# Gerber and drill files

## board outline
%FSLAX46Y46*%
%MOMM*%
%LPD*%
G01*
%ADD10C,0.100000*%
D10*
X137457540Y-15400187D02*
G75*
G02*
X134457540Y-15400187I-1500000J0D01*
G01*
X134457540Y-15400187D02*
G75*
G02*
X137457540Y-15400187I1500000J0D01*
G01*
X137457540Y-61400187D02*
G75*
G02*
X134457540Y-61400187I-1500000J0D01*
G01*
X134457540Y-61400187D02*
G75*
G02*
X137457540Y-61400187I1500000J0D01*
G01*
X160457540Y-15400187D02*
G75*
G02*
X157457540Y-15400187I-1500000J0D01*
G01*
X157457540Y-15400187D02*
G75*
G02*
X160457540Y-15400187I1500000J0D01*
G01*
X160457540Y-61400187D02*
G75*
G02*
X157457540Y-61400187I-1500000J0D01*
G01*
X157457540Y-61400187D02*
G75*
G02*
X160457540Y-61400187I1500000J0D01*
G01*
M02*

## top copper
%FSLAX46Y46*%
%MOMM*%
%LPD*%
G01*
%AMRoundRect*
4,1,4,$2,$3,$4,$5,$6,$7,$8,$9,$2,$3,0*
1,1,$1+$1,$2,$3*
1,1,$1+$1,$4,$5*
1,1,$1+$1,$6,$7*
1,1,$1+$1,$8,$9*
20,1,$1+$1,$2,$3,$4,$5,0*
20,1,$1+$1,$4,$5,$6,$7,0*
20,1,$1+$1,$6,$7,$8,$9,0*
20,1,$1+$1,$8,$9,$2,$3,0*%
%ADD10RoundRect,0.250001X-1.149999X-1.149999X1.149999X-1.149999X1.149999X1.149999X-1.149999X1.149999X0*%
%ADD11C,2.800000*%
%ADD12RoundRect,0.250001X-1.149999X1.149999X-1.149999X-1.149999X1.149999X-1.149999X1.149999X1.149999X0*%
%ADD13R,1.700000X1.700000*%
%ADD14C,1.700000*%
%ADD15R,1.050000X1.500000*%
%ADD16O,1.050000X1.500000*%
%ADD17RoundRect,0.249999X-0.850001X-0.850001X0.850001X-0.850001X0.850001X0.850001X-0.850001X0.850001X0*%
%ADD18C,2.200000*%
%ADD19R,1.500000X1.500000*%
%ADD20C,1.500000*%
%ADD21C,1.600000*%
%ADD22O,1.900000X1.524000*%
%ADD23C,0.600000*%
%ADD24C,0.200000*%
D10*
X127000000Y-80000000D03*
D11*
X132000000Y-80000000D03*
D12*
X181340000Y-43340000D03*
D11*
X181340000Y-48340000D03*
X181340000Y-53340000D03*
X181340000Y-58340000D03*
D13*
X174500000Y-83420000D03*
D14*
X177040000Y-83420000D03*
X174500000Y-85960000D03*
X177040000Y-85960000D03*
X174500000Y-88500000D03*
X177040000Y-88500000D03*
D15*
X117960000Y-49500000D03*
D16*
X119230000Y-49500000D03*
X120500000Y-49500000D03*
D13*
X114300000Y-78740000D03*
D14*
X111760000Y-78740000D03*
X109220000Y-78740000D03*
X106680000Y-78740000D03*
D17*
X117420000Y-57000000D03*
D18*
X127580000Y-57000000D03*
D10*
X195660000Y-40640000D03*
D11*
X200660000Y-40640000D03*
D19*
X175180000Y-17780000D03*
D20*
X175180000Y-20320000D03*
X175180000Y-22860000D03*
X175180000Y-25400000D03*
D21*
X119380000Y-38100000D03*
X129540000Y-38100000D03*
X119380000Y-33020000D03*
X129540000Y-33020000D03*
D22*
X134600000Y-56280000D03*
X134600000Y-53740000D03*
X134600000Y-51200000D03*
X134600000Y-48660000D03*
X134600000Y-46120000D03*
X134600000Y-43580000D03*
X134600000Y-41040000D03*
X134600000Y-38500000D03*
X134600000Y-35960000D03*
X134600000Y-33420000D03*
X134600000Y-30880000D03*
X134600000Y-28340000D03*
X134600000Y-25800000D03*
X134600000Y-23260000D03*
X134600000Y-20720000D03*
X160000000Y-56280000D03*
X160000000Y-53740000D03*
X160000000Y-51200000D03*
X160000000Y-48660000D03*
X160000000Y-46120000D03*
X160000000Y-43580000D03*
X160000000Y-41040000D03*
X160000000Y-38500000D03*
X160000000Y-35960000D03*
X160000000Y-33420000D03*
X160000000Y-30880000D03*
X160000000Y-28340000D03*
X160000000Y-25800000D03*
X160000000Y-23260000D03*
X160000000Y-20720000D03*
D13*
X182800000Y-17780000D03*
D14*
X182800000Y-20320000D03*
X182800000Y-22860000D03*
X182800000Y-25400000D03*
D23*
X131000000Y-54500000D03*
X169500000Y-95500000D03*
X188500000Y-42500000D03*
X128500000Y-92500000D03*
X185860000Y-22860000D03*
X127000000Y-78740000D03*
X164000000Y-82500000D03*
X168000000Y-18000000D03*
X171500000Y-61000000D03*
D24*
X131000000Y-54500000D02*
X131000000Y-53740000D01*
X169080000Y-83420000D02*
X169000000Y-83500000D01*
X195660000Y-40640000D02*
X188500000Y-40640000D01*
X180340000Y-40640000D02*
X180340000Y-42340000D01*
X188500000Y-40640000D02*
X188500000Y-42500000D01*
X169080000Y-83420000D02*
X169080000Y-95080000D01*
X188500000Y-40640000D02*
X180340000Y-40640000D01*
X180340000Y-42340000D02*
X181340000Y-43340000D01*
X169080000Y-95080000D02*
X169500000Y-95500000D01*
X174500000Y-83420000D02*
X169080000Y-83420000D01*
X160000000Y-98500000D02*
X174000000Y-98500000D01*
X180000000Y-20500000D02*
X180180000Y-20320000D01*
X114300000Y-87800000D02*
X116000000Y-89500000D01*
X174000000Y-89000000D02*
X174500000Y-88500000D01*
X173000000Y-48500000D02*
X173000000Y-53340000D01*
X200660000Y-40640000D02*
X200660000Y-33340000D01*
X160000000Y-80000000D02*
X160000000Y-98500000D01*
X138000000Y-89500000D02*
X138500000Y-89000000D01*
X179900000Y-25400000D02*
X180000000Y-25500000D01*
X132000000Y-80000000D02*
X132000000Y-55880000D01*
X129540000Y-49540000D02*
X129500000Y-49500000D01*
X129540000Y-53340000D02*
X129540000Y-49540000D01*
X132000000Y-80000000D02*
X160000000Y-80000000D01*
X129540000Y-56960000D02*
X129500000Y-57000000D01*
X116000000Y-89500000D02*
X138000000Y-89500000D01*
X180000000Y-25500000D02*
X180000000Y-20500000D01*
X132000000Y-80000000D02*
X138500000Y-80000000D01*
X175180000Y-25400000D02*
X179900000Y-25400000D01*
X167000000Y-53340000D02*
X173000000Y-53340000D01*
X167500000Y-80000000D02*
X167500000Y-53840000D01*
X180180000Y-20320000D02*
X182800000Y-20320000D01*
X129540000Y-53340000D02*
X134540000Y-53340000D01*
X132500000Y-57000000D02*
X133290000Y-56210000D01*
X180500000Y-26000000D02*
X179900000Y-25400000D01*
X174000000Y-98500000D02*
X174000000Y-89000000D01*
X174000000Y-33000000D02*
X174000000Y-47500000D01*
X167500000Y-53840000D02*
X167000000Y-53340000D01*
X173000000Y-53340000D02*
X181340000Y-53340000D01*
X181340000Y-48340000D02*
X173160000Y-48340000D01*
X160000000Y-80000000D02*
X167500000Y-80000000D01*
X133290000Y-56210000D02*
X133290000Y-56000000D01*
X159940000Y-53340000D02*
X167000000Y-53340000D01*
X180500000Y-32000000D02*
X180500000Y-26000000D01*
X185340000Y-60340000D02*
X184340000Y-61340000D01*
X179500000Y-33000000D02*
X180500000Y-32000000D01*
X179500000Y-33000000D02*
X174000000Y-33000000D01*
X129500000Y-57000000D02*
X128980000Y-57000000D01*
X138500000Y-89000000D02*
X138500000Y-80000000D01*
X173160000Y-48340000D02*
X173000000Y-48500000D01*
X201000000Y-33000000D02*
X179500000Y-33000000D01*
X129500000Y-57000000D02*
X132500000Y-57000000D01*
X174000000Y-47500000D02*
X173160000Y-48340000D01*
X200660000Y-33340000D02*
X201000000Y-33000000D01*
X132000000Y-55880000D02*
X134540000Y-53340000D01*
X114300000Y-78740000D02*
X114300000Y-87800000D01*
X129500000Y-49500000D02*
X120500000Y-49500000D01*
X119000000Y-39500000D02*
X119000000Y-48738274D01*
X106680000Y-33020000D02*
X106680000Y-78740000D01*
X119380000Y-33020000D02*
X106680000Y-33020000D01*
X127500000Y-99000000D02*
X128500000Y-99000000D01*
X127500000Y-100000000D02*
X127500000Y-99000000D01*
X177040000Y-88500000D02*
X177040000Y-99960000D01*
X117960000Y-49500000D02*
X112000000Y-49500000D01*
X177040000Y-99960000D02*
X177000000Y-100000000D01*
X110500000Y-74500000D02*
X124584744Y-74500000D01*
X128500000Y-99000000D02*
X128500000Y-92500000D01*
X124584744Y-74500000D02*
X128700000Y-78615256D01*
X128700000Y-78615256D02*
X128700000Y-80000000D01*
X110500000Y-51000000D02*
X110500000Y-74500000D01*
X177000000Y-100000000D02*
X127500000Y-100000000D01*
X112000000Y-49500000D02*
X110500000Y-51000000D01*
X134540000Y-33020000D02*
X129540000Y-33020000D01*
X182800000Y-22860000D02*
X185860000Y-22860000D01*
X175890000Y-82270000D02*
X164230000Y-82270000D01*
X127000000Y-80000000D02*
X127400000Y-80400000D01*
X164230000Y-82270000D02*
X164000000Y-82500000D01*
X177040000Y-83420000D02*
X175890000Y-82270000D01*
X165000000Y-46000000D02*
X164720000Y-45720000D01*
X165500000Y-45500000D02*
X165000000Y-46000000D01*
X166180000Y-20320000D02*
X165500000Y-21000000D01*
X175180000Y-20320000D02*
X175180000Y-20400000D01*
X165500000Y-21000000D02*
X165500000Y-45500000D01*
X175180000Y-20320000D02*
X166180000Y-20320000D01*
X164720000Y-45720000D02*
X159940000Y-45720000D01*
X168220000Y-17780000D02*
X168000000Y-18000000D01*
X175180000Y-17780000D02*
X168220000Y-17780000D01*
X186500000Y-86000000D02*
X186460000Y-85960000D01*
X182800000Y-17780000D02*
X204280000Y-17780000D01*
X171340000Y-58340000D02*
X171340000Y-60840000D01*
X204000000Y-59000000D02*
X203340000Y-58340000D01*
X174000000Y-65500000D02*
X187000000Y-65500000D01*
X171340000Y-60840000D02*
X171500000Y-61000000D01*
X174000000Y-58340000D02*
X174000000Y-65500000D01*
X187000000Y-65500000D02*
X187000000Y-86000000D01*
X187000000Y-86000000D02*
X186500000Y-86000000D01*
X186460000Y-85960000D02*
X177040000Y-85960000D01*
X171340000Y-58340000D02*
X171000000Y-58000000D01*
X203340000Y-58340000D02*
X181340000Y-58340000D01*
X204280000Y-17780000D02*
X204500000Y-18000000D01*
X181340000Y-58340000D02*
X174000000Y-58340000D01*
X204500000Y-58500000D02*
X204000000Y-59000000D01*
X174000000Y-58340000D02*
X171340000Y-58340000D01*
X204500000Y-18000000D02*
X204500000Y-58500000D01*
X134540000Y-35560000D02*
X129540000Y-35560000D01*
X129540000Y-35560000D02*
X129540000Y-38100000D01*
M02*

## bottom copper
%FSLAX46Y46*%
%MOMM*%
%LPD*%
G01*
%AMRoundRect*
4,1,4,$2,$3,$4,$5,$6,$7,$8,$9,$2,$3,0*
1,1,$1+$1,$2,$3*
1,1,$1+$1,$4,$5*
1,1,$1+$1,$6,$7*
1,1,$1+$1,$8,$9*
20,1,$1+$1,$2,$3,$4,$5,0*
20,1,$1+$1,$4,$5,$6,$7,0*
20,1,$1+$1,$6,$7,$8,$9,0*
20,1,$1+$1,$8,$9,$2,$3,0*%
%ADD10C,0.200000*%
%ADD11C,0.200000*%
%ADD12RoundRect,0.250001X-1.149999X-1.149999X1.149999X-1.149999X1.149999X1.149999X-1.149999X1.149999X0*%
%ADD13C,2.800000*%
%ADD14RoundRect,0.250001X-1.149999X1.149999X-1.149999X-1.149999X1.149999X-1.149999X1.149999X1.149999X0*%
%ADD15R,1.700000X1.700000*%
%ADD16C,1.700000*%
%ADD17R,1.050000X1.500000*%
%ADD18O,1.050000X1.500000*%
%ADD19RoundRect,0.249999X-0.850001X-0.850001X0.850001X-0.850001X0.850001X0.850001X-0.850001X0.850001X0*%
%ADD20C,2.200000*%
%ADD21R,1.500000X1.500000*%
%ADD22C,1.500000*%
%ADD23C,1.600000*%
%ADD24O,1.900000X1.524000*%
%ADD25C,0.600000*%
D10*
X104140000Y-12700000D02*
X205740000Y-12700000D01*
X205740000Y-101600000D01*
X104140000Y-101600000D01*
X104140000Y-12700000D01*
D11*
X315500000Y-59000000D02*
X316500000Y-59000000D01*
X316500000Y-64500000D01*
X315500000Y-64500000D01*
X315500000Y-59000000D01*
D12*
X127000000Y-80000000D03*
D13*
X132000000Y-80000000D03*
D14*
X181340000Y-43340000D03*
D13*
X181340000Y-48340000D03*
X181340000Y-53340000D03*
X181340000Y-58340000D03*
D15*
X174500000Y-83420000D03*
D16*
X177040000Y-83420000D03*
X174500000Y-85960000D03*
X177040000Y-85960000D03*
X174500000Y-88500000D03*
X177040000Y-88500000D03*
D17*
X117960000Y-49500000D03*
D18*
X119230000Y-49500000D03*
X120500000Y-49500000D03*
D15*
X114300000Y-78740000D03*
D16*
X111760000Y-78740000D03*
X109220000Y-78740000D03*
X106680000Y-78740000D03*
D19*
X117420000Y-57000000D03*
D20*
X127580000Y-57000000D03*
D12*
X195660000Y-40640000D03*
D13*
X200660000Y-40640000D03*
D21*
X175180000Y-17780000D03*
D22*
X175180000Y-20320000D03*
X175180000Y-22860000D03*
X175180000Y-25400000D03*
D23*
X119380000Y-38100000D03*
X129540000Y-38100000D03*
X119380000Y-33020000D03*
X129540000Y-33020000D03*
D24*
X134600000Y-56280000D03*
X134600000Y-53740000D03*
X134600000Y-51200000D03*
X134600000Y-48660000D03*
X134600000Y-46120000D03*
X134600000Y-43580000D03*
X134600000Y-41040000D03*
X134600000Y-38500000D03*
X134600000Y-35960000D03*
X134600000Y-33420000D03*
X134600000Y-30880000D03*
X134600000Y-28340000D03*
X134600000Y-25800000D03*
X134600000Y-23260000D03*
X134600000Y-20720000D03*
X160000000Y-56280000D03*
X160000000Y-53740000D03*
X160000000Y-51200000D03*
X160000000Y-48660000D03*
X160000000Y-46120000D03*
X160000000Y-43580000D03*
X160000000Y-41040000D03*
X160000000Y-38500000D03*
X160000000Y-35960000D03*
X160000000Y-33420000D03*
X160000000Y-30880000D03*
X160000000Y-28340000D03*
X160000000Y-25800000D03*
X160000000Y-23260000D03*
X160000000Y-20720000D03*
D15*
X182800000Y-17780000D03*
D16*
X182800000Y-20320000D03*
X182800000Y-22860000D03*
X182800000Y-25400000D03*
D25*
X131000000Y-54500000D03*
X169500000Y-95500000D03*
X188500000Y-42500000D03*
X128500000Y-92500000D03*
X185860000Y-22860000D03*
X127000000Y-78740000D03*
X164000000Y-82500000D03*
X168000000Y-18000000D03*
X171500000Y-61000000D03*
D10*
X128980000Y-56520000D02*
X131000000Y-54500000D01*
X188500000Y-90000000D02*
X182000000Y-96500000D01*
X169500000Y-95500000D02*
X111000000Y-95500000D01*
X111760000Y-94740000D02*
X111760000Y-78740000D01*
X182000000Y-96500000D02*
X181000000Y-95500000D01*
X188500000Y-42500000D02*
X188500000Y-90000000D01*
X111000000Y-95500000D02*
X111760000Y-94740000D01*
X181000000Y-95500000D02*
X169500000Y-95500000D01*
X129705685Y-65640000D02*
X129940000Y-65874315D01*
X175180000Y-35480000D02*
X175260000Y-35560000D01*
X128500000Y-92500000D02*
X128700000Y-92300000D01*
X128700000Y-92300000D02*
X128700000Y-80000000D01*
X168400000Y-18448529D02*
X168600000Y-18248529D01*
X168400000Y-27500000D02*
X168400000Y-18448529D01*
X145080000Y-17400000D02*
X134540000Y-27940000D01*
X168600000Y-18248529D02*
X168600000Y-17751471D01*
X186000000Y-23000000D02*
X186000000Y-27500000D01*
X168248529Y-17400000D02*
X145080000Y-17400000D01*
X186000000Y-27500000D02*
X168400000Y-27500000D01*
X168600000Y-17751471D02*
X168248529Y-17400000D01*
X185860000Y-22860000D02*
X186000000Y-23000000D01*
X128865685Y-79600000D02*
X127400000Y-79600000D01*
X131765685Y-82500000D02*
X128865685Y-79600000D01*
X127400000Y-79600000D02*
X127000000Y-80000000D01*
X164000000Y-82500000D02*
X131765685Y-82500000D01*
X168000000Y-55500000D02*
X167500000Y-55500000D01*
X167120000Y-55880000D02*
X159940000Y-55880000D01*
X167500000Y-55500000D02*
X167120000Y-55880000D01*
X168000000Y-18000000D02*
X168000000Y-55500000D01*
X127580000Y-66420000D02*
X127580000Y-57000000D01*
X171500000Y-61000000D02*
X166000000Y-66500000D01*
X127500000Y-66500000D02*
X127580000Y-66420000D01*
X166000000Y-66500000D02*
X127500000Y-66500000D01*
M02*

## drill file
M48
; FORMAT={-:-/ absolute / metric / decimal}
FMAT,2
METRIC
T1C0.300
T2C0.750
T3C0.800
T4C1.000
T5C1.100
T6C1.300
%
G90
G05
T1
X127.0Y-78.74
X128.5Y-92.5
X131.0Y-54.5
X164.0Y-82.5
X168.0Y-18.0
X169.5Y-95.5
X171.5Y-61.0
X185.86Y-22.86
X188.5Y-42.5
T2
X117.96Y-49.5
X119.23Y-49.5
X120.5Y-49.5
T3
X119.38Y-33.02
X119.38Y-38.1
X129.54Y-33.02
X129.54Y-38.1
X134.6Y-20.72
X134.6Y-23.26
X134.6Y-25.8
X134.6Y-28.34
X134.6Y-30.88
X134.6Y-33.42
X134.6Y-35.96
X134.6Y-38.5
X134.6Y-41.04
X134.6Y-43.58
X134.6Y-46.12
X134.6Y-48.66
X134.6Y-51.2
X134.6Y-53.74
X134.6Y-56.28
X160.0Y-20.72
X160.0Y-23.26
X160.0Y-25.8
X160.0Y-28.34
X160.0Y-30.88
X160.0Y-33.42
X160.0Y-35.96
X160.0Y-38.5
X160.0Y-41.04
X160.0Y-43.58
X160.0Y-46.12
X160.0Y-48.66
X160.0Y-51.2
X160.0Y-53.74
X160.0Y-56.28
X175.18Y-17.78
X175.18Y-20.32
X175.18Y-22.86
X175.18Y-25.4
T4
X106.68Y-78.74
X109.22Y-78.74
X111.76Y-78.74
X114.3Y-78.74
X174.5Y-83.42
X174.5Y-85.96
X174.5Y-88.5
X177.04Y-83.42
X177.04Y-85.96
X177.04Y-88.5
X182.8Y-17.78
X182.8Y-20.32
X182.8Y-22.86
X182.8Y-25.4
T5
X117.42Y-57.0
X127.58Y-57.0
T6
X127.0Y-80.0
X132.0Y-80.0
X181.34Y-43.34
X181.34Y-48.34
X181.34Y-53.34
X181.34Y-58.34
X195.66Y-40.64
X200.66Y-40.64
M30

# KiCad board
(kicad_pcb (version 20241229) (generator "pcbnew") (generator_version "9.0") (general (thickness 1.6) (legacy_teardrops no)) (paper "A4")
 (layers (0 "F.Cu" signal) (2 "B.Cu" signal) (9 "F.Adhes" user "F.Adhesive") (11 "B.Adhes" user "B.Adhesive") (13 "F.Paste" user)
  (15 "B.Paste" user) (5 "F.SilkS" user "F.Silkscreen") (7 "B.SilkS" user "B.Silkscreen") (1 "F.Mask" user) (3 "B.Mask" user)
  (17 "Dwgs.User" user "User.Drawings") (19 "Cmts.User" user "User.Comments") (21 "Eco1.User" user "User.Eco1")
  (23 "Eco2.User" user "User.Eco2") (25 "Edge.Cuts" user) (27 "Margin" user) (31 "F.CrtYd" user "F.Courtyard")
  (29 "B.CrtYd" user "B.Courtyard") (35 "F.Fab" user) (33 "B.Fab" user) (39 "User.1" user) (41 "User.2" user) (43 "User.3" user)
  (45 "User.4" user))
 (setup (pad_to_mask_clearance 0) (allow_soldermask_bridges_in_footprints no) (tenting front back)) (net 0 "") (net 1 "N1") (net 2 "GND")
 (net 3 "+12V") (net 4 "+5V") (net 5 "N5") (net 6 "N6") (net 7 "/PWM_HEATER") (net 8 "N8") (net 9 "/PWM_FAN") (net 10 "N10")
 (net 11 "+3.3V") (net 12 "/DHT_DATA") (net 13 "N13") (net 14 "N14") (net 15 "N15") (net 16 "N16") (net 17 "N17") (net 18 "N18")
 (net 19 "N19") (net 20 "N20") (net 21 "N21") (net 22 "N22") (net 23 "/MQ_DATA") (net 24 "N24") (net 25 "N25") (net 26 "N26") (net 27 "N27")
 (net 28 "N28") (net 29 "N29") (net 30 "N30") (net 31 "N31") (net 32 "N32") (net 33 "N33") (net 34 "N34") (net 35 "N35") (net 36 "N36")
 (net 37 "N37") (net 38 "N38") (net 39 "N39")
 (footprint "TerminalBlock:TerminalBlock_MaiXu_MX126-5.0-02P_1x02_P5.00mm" (layer "F.Cu") (at 127 80)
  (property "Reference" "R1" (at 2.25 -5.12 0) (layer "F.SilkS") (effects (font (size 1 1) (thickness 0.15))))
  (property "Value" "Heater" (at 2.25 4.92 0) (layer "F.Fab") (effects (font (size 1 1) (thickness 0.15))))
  (pad "1" thru_hole roundrect (at 0 0) (size 2.8 2.8) (drill 1.3) (layers "*.Cu" "*.Mask") (remove_unused_layers no)
   (roundrect_rratio 0.089286) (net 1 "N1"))
  (pad "2" thru_hole circle (at 5 0) (size 2.8 2.8) (drill 1.3) (layers "*.Cu" "*.Mask") (remove_unused_layers no) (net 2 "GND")))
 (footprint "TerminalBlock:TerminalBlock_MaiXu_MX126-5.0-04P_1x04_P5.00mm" (layer "F.Cu") (at 181.34 43.34 -90)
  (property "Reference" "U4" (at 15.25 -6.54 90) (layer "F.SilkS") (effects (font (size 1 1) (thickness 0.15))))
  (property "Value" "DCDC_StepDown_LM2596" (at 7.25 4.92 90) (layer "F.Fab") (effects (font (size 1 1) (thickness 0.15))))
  (pad "1" thru_hole roundrect (at 0 0 270) (size 2.8 2.8) (drill 1.3) (layers "*.Cu" "*.Mask") (remove_unused_layers no)
   (roundrect_rratio 0.089286) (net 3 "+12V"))
  (pad "2" thru_hole circle (at 5 0 270) (size 2.8 2.8) (drill 1.3) (layers "*.Cu" "*.Mask") (remove_unused_layers no) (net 2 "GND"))
  (pad "3" thru_hole circle (at 10 0 270) (size 2.8 2.8) (drill 1.3) (layers "*.Cu" "*.Mask") (remove_unused_layers no) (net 2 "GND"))
  (pad "4" thru_hole circle (at 15 0 270) (size 2.8 2.8) (drill 1.3) (layers "*.Cu" "*.Mask") (remove_unused_layers no) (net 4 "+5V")))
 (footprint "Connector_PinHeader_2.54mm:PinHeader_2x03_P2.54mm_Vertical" (layer "F.Cu") (at 174.5 83.42)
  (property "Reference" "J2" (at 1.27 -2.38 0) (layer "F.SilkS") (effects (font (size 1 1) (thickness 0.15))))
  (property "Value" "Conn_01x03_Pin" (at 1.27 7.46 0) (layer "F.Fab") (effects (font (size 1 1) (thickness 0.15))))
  (pad "1" thru_hole rect (at 0 0) (size 1.7 1.7) (drill 1) (layers "*.Cu" "*.Mask") (remove_unused_layers no) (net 3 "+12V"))
  (pad "2" thru_hole circle (at 2.54 0) (size 1.7 1.7) (drill 1) (layers "*.Cu" "*.Mask") (remove_unused_layers no) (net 1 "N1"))
  (pad "3" thru_hole circle (at 0 2.54) (size 1.7 1.7) (drill 1) (layers "*.Cu" "*.Mask") (remove_unused_layers no) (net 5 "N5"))
  (pad "4" thru_hole circle (at 2.54 2.54) (size 1.7 1.7) (drill 1) (layers "*.Cu" "*.Mask") (remove_unused_layers no) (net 4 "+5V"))
  (pad "5" thru_hole circle (at 0 5.08) (size 1.7 1.7) (drill 1) (layers "*.Cu" "*.Mask") (remove_unused_layers no) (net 2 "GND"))
  (pad "6" thru_hole circle (at 2.54 5.08) (size 1.7 1.7) (drill 1) (layers "*.Cu" "*.Mask") (remove_unused_layers no) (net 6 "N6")))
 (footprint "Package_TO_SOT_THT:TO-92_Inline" (layer "F.Cu") (at 117.96 49.5)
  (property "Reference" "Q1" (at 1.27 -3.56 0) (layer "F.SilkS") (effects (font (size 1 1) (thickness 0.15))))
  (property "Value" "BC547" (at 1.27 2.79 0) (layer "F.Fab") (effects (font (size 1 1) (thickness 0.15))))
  (pad "1" thru_hole rect (at 0 0) (size 1.05 1.5) (drill 0.75) (layers "*.Cu" "*.Mask") (remove_unused_layers no) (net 6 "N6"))
  (pad "2" thru_hole oval (at 1.27 0) (size 1.05 1.5) (drill 0.75) (layers "*.Cu" "*.Mask") (remove_unused_layers no) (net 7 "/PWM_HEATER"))
  (pad "3" thru_hole oval (at 2.54 0) (size 1.05 1.5) (drill 0.75) (layers "*.Cu" "*.Mask") (remove_unused_layers no) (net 2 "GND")))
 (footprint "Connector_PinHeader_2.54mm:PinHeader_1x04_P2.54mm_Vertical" (layer "F.Cu") (at 114.3 78.74 -90)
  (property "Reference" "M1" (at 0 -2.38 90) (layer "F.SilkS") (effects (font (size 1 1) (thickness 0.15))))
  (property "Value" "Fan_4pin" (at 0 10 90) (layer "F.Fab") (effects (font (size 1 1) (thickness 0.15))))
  (pad "1" thru_hole rect (at 0 0 270) (size 1.7 1.7) (drill 1) (layers "*.Cu" "*.Mask") (remove_unused_layers no) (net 2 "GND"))
  (pad "2" thru_hole circle (at 0 2.54 270) (size 1.7 1.7) (drill 1) (layers "*.Cu" "*.Mask") (remove_unused_layers no) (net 3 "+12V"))
  (pad "3" thru_hole circle (at 0 5.08 270) (size 1.7 1.7) (drill 1) (layers "*.Cu" "*.Mask") (remove_unused_layers no) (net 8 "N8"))
  (pad "4" thru_hole circle (at 0 7.62 270) (size 1.7 1.7) (drill 1) (layers "*.Cu" "*.Mask") (remove_unused_layers no) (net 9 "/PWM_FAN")))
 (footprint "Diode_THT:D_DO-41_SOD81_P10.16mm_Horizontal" (layer "F.Cu") (at 117.42 57)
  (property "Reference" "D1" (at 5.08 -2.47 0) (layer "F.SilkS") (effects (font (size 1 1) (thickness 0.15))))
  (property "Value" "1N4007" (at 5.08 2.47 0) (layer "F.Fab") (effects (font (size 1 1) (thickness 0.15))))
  (pad "1" thru_hole roundrect (at 0 0) (size 2.2 2.2) (drill 1.1) (layers "*.Cu" "*.Mask") (remove_unused_layers no)
   (roundrect_rratio 0.113636) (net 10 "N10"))
  (pad "2" thru_hole circle (at 10.16 0) (size 2.2 2.2) (drill 1.1) (layers "*.Cu" "*.Mask") (remove_unused_layers no) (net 4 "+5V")))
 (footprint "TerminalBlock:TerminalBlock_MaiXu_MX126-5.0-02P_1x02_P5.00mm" (layer "F.Cu") (at 195.66 40.64)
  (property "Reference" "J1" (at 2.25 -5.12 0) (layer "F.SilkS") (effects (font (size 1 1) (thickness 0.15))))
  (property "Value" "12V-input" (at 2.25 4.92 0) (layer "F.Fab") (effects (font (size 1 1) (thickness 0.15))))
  (pad "1" thru_hole roundrect (at 0 0) (size 2.8 2.8) (drill 1.3) (layers "*.Cu" "*.Mask") (remove_unused_layers no)
   (roundrect_rratio 0.089286) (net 3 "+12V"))
  (pad "2" thru_hole circle (at 5 0) (size 2.8 2.8) (drill 1.3) (layers "*.Cu" "*.Mask") (remove_unused_layers no) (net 2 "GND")))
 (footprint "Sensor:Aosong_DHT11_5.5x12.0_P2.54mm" (layer "F.Cu") (at 175.18 17.78)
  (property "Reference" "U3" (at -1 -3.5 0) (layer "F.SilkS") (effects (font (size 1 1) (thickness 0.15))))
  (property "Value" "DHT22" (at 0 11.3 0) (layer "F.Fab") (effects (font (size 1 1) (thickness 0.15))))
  (pad "1" thru_hole rect (at 0 0) (size 1.5 1.5) (drill 0.8) (layers "*.Cu" "*.Mask") (remove_unused_layers no) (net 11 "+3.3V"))
  (pad "2" thru_hole circle (at 0 2.54) (size 1.5 1.5) (drill 0.8) (layers "*.Cu" "*.Mask") (remove_unused_layers no) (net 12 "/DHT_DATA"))
  (pad "3" thru_hole circle (at 0 5.08) (size 1.5 1.5) (drill 0.8) (layers "*.Cu" "*.Mask") (remove_unused_layers no) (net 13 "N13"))
  (pad "4" thru_hole circle (at 0 7.62) (size 1.5 1.5) (drill 0.8) (layers "*.Cu" "*.Mask") (remove_unused_layers no) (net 2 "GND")))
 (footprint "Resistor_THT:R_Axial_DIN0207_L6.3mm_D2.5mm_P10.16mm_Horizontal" (layer "F.Cu") (at 119.38 38.1)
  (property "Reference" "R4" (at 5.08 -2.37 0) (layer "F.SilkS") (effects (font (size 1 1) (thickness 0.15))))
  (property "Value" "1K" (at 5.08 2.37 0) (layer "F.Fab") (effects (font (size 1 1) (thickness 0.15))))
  (pad "1" thru_hole circle (at 0 0) (size 1.6 1.6) (drill 0.8) (layers "*.Cu" "*.Mask") (remove_unused_layers no) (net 7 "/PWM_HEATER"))
  (pad "2" thru_hole circle (at 10.16 0) (size 1.6 1.6) (drill 0.8) (layers "*.Cu" "*.Mask") (remove_unused_layers no) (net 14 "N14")))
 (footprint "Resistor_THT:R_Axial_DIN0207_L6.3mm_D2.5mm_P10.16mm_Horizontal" (layer "F.Cu") (at 119.38 33.02)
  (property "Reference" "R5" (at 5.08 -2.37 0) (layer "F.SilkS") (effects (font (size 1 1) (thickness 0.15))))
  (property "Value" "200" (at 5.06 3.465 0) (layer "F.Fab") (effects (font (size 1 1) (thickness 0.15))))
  (pad "1" thru_hole circle (at 0 0) (size 1.6 1.6) (drill 0.8) (layers "*.Cu" "*.Mask") (remove_unused_layers no) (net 9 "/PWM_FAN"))
  (pad "2" thru_hole circle (at 10.16 0) (size 1.6 1.6) (drill 0.8) (layers "*.Cu" "*.Mask") (remove_unused_layers no) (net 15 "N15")))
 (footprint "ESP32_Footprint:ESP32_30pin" (layer "F.Cu") (at 146.52754 39.260187)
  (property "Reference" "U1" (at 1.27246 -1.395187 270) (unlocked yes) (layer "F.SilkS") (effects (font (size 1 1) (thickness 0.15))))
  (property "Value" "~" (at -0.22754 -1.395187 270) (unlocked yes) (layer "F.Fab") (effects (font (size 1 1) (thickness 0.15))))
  (fp_circle (center -10.57 -23.86) (end -10.57 -22.36) (stroke (width 0.1) (type default)) (fill no) (layer "Edge.Cuts"))
  (fp_circle (center -10.57 22.14) (end -10.57 23.64) (stroke (width 0.1) (type default)) (fill no) (layer "Edge.Cuts"))
  (fp_circle (center 12.43 -23.86) (end 12.43 -22.36) (stroke (width 0.1) (type default)) (fill no) (layer "Edge.Cuts"))
  (fp_circle (center 12.43 22.14) (end 12.43 23.64) (stroke (width 0.1) (type default)) (fill no) (layer "Edge.Cuts"))
  (pad "1" thru_hole oval (at -11.92754 17.019813 270) (size 1.524 1.9) (drill 0.8) (layers "*.Cu" "*.Mask") (remove_unused_layers no)
   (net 10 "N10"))
  (pad "2" thru_hole oval (at -11.92754 14.479813 270) (size 1.524 1.9) (drill 0.8) (layers "*.Cu" "*.Mask") (remove_unused_layers no)
   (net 2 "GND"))
  (pad "3" thru_hole oval (at -11.92754 11.939813 270) (size 1.524 1.9) (drill 0.8) (layers "*.Cu" "*.Mask") (remove_unused_layers no)
   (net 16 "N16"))
  (pad "4" thru_hole oval (at -11.92754 9.399813 270) (size 1.524 1.9) (drill 0.8) (layers "*.Cu" "*.Mask") (remove_unused_layers no)
   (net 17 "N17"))
  (pad "5" thru_hole oval (at -11.92754 6.859813 270) (size 1.524 1.9) (drill 0.8) (layers "*.Cu" "*.Mask") (remove_unused_layers no)
   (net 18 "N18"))
  (pad "6" thru_hole oval (at -11.92754 4.319813 270) (size 1.524 1.9) (drill 0.8) (layers "*.Cu" "*.Mask") (remove_unused_layers no)
   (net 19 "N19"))
  (pad "7" thru_hole oval (at -11.92754 1.779813 270) (size 1.524 1.9) (drill 0.8) (layers "*.Cu" "*.Mask") (remove_unused_layers no)
   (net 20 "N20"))
  (pad "8" thru_hole oval (at -11.92754 -0.760187 270) (size 1.524 1.9) (drill 0.8) (layers "*.Cu" "*.Mask") (remove_unused_layers no)
   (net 14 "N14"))
  (pad "9" thru_hole oval (at -11.92754 -3.300187 270) (size 1.524 1.9) (drill 0.8) (layers "*.Cu" "*.Mask") (remove_unused_layers no)
   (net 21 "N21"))
  (pad "10" thru_hole oval (at -11.92754 -5.840187 270) (size 1.524 1.9) (drill 0.8) (layers "*.Cu" "*.Mask") (remove_unused_layers no)
   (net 15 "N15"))
  (pad "11" thru_hole oval (at -11.92754 -8.380187 270) (size 1.524 1.9) (drill 0.8) (layers "*.Cu" "*.Mask") (remove_unused_layers no)
   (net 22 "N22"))
  (pad "12" thru_hole oval (at -11.92754 -10.920187 270) (size 1.524 1.9) (drill 0.8) (layers "*.Cu" "*.Mask") (remove_unused_layers no)
   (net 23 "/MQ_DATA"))
  (pad "13" thru_hole oval (at -11.92754 -13.460187 270) (size 1.524 1.9) (drill 0.8) (layers "*.Cu" "*.Mask") (remove_unused_layers no)
   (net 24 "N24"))
  (pad "14" thru_hole oval (at -11.92754 -16.000187 270) (size 1.524 1.9) (drill 0.8) (layers "*.Cu" "*.Mask") (remove_unused_layers no)
   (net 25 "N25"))
  (pad "15" thru_hole oval (at -11.92754 -18.540187 270) (size 1.524 1.9) (drill 0.8) (layers "*.Cu" "*.Mask") (remove_unused_layers no)
   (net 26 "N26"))
  (pad "16" thru_hole oval (at 13.47246 17.019813 270) (size 1.524 1.9) (drill 0.8) (layers "*.Cu" "*.Mask") (remove_unused_layers no)
   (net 11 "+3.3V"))
  (pad "17" thru_hole oval (at 13.47246 14.479813 270) (size 1.524 1.9) (drill 0.8) (layers "*.Cu" "*.Mask") (remove_unused_layers no)
   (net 2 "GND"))
  (pad "18" thru_hole oval (at 13.47246 11.939813 270) (size 1.524 1.9) (drill 0.8) (layers "*.Cu" "*.Mask") (remove_unused_layers no)
   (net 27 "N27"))
  (pad "19" thru_hole oval (at 13.47246 9.399813 270) (size 1.524 1.9) (drill 0.8) (layers "*.Cu" "*.Mask") (remove_unused_layers no)
   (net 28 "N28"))
  (pad "20" thru_hole oval (at 13.47246 6.859813 270) (size 1.524 1.9) (drill 0.8) (layers "*.Cu" "*.Mask" "Dwgs.User")
   (remove_unused_layers no) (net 12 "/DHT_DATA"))
  (pad "21" thru_hole oval (at 13.47246 4.319813 270) (size 1.524 1.9) (drill 0.8) (layers "*.Cu" "*.Mask") (remove_unused_layers no)
   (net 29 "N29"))
  (pad "22" thru_hole oval (at 13.47246 1.779813 270) (size 1.524 1.9) (drill 0.8) (layers "*.Cu" "*.Mask") (remove_unused_layers no)
   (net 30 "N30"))
  (pad "23" thru_hole oval (at 13.47246 -0.760187 270) (size 1.524 1.9) (drill 0.8) (layers "*.Cu" "*.Mask") (remove_unused_layers no)
   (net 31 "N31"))
  (pad "24" thru_hole oval (at 13.47246 -3.300187 270) (size 1.524 1.9) (drill 0.8) (layers "*.Cu" "*.Mask") (remove_unused_layers no)
   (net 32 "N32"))
  (pad "25" thru_hole oval (at 13.47246 -5.840187 270) (size 1.524 1.9) (drill 0.8) (layers "*.Cu" "*.Mask") (remove_unused_layers no)
   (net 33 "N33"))
  (pad "26" thru_hole oval (at 13.47246 -8.380187 270) (size 1.524 1.9) (drill 0.8) (layers "*.Cu" "*.Mask") (remove_unused_layers no)
   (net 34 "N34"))
  (pad "27" thru_hole oval (at 13.47246 -10.920187 270) (size 1.524 1.9) (drill 0.8) (layers "*.Cu" "*.Mask") (remove_unused_layers no)
   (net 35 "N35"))
  (pad "28" thru_hole oval (at 13.47246 -13.460187 270) (size 1.524 1.9) (drill 0.8) (layers "*.Cu" "*.Mask") (remove_unused_layers no)
   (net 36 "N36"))
  (pad "29" thru_hole oval (at 13.47246 -16.000187 270) (size 1.524 1.9) (drill 0.8) (layers "*.Cu" "*.Mask") (remove_unused_layers no)
   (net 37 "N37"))
  (pad "30" thru_hole oval (at 13.47246 -18.540187 270) (size 1.524 1.9) (drill 0.8) (layers "*.Cu" "*.Mask") (remove_unused_layers no)
   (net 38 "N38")))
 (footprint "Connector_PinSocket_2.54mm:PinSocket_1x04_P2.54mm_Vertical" (layer "F.Cu") (at 182.8 17.78)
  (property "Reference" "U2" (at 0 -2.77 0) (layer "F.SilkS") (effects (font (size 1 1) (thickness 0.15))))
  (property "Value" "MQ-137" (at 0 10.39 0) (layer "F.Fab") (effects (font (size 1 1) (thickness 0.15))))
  (pad "1" thru_hole rect (at 0 0) (size 1.7 1.7) (drill 1) (layers "*.Cu" "*.Mask") (remove_unused_layers no) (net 4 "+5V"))
  (pad "2" thru_hole circle (at 0 2.54) (size 1.7 1.7) (drill 1) (layers "*.Cu" "*.Mask") (remove_unused_layers no) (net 2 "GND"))
  (pad "3" thru_hole circle (at 0 5.08) (size 1.7 1.7) (drill 1) (layers "*.Cu" "*.Mask") (remove_unused_layers no) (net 23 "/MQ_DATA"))
  (pad "4" thru_hole circle (at 0 7.62) (size 1.7 1.7) (drill 1) (layers "*.Cu" "*.Mask") (remove_unused_layers no) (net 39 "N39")))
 (gr_rect (start 104.14 12.7) (end 205.74 101.6) (stroke (width 0.2) (type default)) (fill no) (layer "B.Cu") (net 9))
 (gr_rect (start 315.5 59) (end 316.5 64.5) (stroke (width 0.2) (type default)) (fill no) (layer "B.Cu"))
 (segment (start 131 54.5) (end 131 53.74) (width 0.2) (layer "F.Cu") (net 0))
 (via (at 131 54.5) (size 0.6) (drill 0.3) (layers "F.Cu" "B.Cu") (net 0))
 (segment (start 128.98 56.52) (end 131 54.5) (width 0.2) (layer "B.Cu") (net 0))
 (segment (start 169.08 83.42) (end 169 83.5) (width 0.2) (layer "F.Cu") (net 3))
 (segment (start 195.66 40.64) (end 188.5 40.64) (width 0.2) (layer "F.Cu") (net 3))
 (segment (start 180.34 40.64) (end 180.34 42.34) (width 0.2) (layer "F.Cu") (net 3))
 (segment (start 188.5 40.64) (end 188.5 42.5) (width 0.2) (layer "F.Cu") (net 3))
 (segment (start 169.08 83.42) (end 169.08 95.08) (width 0.2) (layer "F.Cu") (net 3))
 (segment (start 188.5 40.64) (end 180.34 40.64) (width 0.2) (layer "F.Cu") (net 3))
 (segment (start 180.34 42.34) (end 181.34 43.34) (width 0.2) (layer "F.Cu") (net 3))
 (segment (start 169.08 95.08) (end 169.5 95.5) (width 0.2) (layer "F.Cu") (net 3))
 (segment (start 174.5 83.42) (end 169.08 83.42) (width 0.2) (layer "F.Cu") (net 3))
 (via (at 169.5 95.5) (size 0.6) (drill 0.3) (layers "F.Cu" "B.Cu") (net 3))
 (via (at 188.5 42.5) (size 0.6) (drill 0.3) (layers "F.Cu" "B.Cu") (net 3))
 (segment (start 188.5 90) (end 182 96.5) (width 0.2) (layer "B.Cu") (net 3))
 (segment (start 169.5 95.5) (end 111 95.5) (width 0.2) (layer "B.Cu") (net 3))
 (segment (start 111.76 94.74) (end 111.76 78.74) (width 0.2) (layer "B.Cu") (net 3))
 (segment (start 182 96.5) (end 181 95.5) (width 0.2) (layer "B.Cu") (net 3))
 (segment (start 188.5 42.5) (end 188.5 90) (width 0.2) (layer "B.Cu") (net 3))
 (segment (start 111 95.5) (end 111.76 94.74) (width 0.2) (layer "B.Cu") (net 3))
 (segment (start 181 95.5) (end 169.5 95.5) (width 0.2) (layer "B.Cu") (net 3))
 (segment (start 160 98.5) (end 174 98.5) (width 0.2) (layer "F.Cu") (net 2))
 (segment (start 180 20.5) (end 180.18 20.32) (width 0.2) (layer "F.Cu") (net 2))
 (segment (start 114.3 87.8) (end 116 89.5) (width 0.2) (layer "F.Cu") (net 2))
 (segment (start 174 89) (end 174.5 88.5) (width 0.2) (layer "F.Cu") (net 2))
 (segment (start 173 48.5) (end 173 53.34) (width 0.2) (layer "F.Cu") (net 2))
 (segment (start 200.66 40.64) (end 200.66 33.34) (width 0.2) (layer "F.Cu") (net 2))
 (segment (start 160 80) (end 160 98.5) (width 0.2) (layer "F.Cu") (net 2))
 (segment (start 138 89.5) (end 138.5 89) (width 0.2) (layer "F.Cu") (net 2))
 (segment (start 179.9 25.4) (end 180 25.5) (width 0.2) (layer "F.Cu") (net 2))
 (segment (start 132 80) (end 132 55.88) (width 0.2) (layer "F.Cu") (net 2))
 (segment (start 129.54 49.54) (end 129.5 49.5) (width 0.2) (layer "F.Cu") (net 2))
 (segment (start 129.54 53.34) (end 129.54 49.54) (width 0.2) (layer "F.Cu") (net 2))
 (segment (start 132 80) (end 160 80) (width 0.2) (layer "F.Cu") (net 2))
 (segment (start 129.54 56.96) (end 129.5 57) (width 0.2) (layer "F.Cu") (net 2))
 (segment (start 116 89.5) (end 138 89.5) (width 0.2) (layer "F.Cu") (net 2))
 (segment (start 180 25.5) (end 180 20.5) (width 0.2) (layer "F.Cu") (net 2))
 (segment (start 132 80) (end 138.5 80) (width 0.2) (layer "F.Cu") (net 2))
 (segment (start 175.18 25.4) (end 179.9 25.4) (width 0.2) (layer "F.Cu") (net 2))
 (segment (start 167 53.34) (end 173 53.34) (width 0.2) (layer "F.Cu") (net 2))
 (segment (start 167.5 80) (end 167.5 53.84) (width 0.2) (layer "F.Cu") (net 2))
 (segment (start 180.18 20.32) (end 182.8 20.32) (width 0.2) (layer "F.Cu") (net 2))
 (segment (start 129.54 53.34) (end 134.54 53.34) (width 0.2) (layer "F.Cu") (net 2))
 (segment (start 132.5 57) (end 133.29 56.21) (width 0.2) (layer "F.Cu") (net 2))
 (segment (start 180.5 26) (end 179.9 25.4) (width 0.2) (layer "F.Cu") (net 2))
 (segment (start 174 98.5) (end 174 89) (width 0.2) (layer "F.Cu") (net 2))
 (segment (start 174 33) (end 174 47.5) (width 0.2) (layer "F.Cu") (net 2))
 (segment (start 167.5 53.84) (end 167 53.34) (width 0.2) (layer "F.Cu") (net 2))
 (segment (start 173 53.34) (end 181.34 53.34) (width 0.2) (layer "F.Cu") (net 2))
 (segment (start 181.34 48.34) (end 173.16 48.34) (width 0.2) (layer "F.Cu") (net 2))
 (segment (start 160 80) (end 167.5 80) (width 0.2) (layer "F.Cu") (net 2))
 (segment (start 133.29 56.21) (end 133.29 56) (width 0.2) (layer "F.Cu") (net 2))
 (segment (start 159.94 53.34) (end 167 53.34) (width 0.2) (layer "F.Cu") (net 2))
 (segment (start 180.5 32) (end 180.5 26) (width 0.2) (layer "F.Cu") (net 2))
 (segment (start 185.34 60.34) (end 184.34 61.34) (width 0.2) (layer "F.Cu") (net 2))
 (segment (start 179.5 33) (end 180.5 32) (width 0.2) (layer "F.Cu") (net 2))
 (segment (start 179.5 33) (end 174 33) (width 0.2) (layer "F.Cu") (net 2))
 (segment (start 129.5 57) (end 128.98 57) (width 0.2) (layer "F.Cu") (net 2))
 (segment (start 138.5 89) (end 138.5 80) (width 0.2) (layer "F.Cu") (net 2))
 (segment (start 173.16 48.34) (end 173 48.5) (width 0.2) (layer "F.Cu") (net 2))
 (segment (start 201 33) (end 179.5 33) (width 0.2) (layer "F.Cu") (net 2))
 (segment (start 129.5 57) (end 132.5 57) (width 0.2) (layer "F.Cu") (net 2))
 (segment (start 174 47.5) (end 173.16 48.34) (width 0.2) (layer "F.Cu") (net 2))
 (segment (start 200.66 33.34) (end 201 33) (width 0.2) (layer "F.Cu") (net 2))
 (segment (start 132 55.88) (end 134.54 53.34) (width 0.2) (layer "F.Cu") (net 2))
 (segment (start 114.3 78.74) (end 114.3 87.8) (width 0.2) (layer "F.Cu") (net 2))
 (segment (start 129.5 49.5) (end 120.5 49.5) (width 0.2) (layer "F.Cu") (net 2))
 (segment (start 129.705685 65.64) (end 129.94 65.874315) (width 0.2) (layer "B.Cu") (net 2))
 (segment (start 175.18 35.48) (end 175.26 35.56) (width 0.2) (layer "B.Cu") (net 2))
 (segment (start 119 39.5) (end 119 48.738274) (width 0.2) (layer "F.Cu") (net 7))
 (segment (start 106.68 33.02) (end 106.68 78.74) (width 0.2) (layer "F.Cu") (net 9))
 (segment (start 119.38 33.02) (end 106.68 33.02) (width 0.2) (layer "F.Cu") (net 9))
 (segment (start 127.5 99) (end 128.5 99) (width 0.2) (layer "F.Cu") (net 6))
 (segment (start 127.5 100) (end 127.5 99) (width 0.2) (layer "F.Cu") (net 6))
 (segment (start 177.04 88.5) (end 177.04 99.96) (width 0.2) (layer "F.Cu") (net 6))
 (segment (start 117.96 49.5) (end 112 49.5) (width 0.2) (layer "F.Cu") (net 6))
 (segment (start 177.04 99.96) (end 177 100) (width 0.2) (layer "F.Cu") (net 6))
 (segment (start 110.5 74.5) (end 124.584744 74.5) (width 0.2) (layer "F.Cu") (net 6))
 (segment (start 128.5 99) (end 128.5 92.5) (width 0.2) (layer "F.Cu") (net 6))
 (segment (start 124.584744 74.5) (end 128.7 78.615256) (width 0.2) (layer "F.Cu") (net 6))
 (segment (start 128.7 78.615256) (end 128.7 80) (width 0.2) (layer "F.Cu") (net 6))
 (segment (start 110.5 51) (end 110.5 74.5) (width 0.2) (layer "F.Cu") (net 6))
 (segment (start 177 100) (end 127.5 100) (width 0.2) (layer "F.Cu") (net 6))
 (segment (start 112 49.5) (end 110.5 51) (width 0.2) (layer "F.Cu") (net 6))
 (via (at 128.5 92.5) (size 0.6) (drill 0.3) (layers "F.Cu" "B.Cu") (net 6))
 (segment (start 128.5 92.5) (end 128.7 92.3) (width 0.2) (layer "B.Cu") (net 6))
 (segment (start 128.7 92.3) (end 128.7 80) (width 0.2) (layer "B.Cu") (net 6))
 (segment (start 134.54 33.02) (end 129.54 33.02) (width 0.2) (layer "F.Cu") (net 15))
 (segment (start 182.8 22.86) (end 185.86 22.86) (width 0.2) (layer "F.Cu") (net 23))
 (via (at 185.86 22.86) (size 0.6) (drill 0.3) (layers "F.Cu" "B.Cu") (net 23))
 (segment (start 168.4 18.448529) (end 168.6 18.248529) (width 0.2) (layer "B.Cu") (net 23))
 (segment (start 168.4 27.5) (end 168.4 18.448529) (width 0.2) (layer "B.Cu") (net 23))
 (segment (start 145.08 17.4) (end 134.54 27.94) (width 0.2) (layer "B.Cu") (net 23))
 (segment (start 168.6 18.248529) (end 168.6 17.751471) (width 0.2) (layer "B.Cu") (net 23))
 (segment (start 186 23) (end 186 27.5) (width 0.2) (layer "B.Cu") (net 23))
 (segment (start 168.248529 17.4) (end 145.08 17.4) (width 0.2) (layer "B.Cu") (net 23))
 (segment (start 186 27.5) (end 168.4 27.5) (width 0.2) (layer "B.Cu") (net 23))
 (segment (start 168.6 17.751471) (end 168.248529 17.4) (width 0.2) (layer "B.Cu") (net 23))
 (segment (start 185.86 22.86) (end 186 23) (width 0.2) (layer "B.Cu") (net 23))
 (segment (start 175.89 82.27) (end 164.23 82.27) (width 0.2) (layer "F.Cu") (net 1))
 (segment (start 127 80) (end 127.4 80.4) (width 0.2) (layer "F.Cu") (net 1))
 (segment (start 164.23 82.27) (end 164 82.5) (width 0.2) (layer "F.Cu") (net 1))
 (segment (start 177.04 83.42) (end 175.89 82.27) (width 0.2) (layer "F.Cu") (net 1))
 (via (at 127 78.74) (size 0.6) (drill 0.3) (layers "F.Cu" "B.Cu") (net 1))
 (via (at 164 82.5) (size 0.6) (drill 0.3) (layers "F.Cu" "B.Cu") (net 1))
 (segment (start 128.865685 79.6) (end 127.4 79.6) (width 0.2) (layer "B.Cu") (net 1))
 (segment (start 131.765685 82.5) (end 128.865685 79.6) (width 0.2) (layer "B.Cu") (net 1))
 (segment (start 127.4 79.6) (end 127 80) (width 0.2) (layer "B.Cu") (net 1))
 (segment (start 164 82.5) (end 131.765685 82.5) (width 0.2) (layer "B.Cu") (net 1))
 (segment (start 165 46) (end 164.72 45.72) (width 0.2) (layer "F.Cu") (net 12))
 (segment (start 165.5 45.5) (end 165 46) (width 0.2) (layer "F.Cu") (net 12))
 (segment (start 166.18 20.32) (end 165.5 21) (width 0.2) (layer "F.Cu") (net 12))
 (segment (start 175.18 20.32) (end 175.18 20.4) (width 0.2) (layer "F.Cu") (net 12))
 (segment (start 165.5 21) (end 165.5 45.5) (width 0.2) (layer "F.Cu") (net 12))
 (segment (start 175.18 20.32) (end 166.18 20.32) (width 0.2) (layer "F.Cu") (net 12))
 (segment (start 164.72 45.72) (end 159.94 45.72) (width 0.2) (layer "F.Cu") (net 12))
 (segment (start 168.22 17.78) (end 168 18) (width 0.2) (layer "F.Cu") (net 11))
 (segment (start 175.18 17.78) (end 168.22 17.78) (width 0.2) (layer "F.Cu") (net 11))
 (via (at 168 18) (size 0.6) (drill 0.3) (layers "F.Cu" "B.Cu") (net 11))
 (segment (start 168 55.5) (end 167.5 55.5) (width 0.2) (layer "B.Cu") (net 11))
 (segment (start 167.12 55.88) (end 159.94 55.88) (width 0.2) (layer "B.Cu") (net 11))
 (segment (start 167.5 55.5) (end 167.12 55.88) (width 0.2) (layer "B.Cu") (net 11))
 (segment (start 168 18) (end 168 55.5) (width 0.2) (layer "B.Cu") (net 11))
 (segment (start 186.5 86) (end 186.46 85.96) (width 0.2) (layer "F.Cu") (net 4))
 (segment (start 182.8 17.78) (end 204.28 17.78) (width 0.2) (layer "F.Cu") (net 4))
 (segment (start 171.34 58.34) (end 171.34 60.84) (width 0.2) (layer "F.Cu") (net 4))
 (segment (start 204 59) (end 203.34 58.34) (width 0.2) (layer "F.Cu") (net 4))
 (segment (start 174 65.5) (end 187 65.5) (width 0.2) (layer "F.Cu") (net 4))
 (segment (start 171.34 60.84) (end 171.5 61) (width 0.2) (layer "F.Cu") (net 4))
 (segment (start 174 58.34) (end 174 65.5) (width 0.2) (layer "F.Cu") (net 4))
 (segment (start 187 65.5) (end 187 86) (width 0.2) (layer "F.Cu") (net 4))
 (segment (start 187 86) (end 186.5 86) (width 0.2) (layer "F.Cu") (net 4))
 (segment (start 186.46 85.96) (end 177.04 85.96) (width 0.2) (layer "F.Cu") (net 4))
 (segment (start 171.34 58.34) (end 171 58) (width 0.2) (layer "F.Cu") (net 4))
 (segment (start 203.34 58.34) (end 181.34 58.34) (width 0.2) (layer "F.Cu") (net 4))
 (segment (start 204.28 17.78) (end 204.5 18) (width 0.2) (layer "F.Cu") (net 4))
 (segment (start 181.34 58.34) (end 174 58.34) (width 0.2) (layer "F.Cu") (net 4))
 (segment (start 204.5 58.5) (end 204 59) (width 0.2) (layer "F.Cu") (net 4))
 (segment (start 174 58.34) (end 171.34 58.34) (width 0.2) (layer "F.Cu") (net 4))
 (segment (start 204.5 18) (end 204.5 58.5) (width 0.2) (layer "F.Cu") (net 4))
 (via (at 171.5 61) (size 0.6) (drill 0.3) (layers "F.Cu" "B.Cu") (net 4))
 (segment (start 127.58 66.42) (end 127.58 57) (width 0.2) (layer "B.Cu") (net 4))
 (segment (start 171.5 61) (end 166 66.5) (width 0.2) (layer "B.Cu") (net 4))
 (segment (start 127.5 66.5) (end 127.58 66.42) (width 0.2) (layer "B.Cu") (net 4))
 (segment (start 166 66.5) (end 127.5 66.5) (width 0.2) (layer "B.Cu") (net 4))
 (segment (start 134.54 35.56) (end 129.54 35.56) (width 0.2) (layer "F.Cu") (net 21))
 (segment (start 129.54 35.56) (end 129.54 38.1) (width 0.2) (layer "F.Cu") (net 21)))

